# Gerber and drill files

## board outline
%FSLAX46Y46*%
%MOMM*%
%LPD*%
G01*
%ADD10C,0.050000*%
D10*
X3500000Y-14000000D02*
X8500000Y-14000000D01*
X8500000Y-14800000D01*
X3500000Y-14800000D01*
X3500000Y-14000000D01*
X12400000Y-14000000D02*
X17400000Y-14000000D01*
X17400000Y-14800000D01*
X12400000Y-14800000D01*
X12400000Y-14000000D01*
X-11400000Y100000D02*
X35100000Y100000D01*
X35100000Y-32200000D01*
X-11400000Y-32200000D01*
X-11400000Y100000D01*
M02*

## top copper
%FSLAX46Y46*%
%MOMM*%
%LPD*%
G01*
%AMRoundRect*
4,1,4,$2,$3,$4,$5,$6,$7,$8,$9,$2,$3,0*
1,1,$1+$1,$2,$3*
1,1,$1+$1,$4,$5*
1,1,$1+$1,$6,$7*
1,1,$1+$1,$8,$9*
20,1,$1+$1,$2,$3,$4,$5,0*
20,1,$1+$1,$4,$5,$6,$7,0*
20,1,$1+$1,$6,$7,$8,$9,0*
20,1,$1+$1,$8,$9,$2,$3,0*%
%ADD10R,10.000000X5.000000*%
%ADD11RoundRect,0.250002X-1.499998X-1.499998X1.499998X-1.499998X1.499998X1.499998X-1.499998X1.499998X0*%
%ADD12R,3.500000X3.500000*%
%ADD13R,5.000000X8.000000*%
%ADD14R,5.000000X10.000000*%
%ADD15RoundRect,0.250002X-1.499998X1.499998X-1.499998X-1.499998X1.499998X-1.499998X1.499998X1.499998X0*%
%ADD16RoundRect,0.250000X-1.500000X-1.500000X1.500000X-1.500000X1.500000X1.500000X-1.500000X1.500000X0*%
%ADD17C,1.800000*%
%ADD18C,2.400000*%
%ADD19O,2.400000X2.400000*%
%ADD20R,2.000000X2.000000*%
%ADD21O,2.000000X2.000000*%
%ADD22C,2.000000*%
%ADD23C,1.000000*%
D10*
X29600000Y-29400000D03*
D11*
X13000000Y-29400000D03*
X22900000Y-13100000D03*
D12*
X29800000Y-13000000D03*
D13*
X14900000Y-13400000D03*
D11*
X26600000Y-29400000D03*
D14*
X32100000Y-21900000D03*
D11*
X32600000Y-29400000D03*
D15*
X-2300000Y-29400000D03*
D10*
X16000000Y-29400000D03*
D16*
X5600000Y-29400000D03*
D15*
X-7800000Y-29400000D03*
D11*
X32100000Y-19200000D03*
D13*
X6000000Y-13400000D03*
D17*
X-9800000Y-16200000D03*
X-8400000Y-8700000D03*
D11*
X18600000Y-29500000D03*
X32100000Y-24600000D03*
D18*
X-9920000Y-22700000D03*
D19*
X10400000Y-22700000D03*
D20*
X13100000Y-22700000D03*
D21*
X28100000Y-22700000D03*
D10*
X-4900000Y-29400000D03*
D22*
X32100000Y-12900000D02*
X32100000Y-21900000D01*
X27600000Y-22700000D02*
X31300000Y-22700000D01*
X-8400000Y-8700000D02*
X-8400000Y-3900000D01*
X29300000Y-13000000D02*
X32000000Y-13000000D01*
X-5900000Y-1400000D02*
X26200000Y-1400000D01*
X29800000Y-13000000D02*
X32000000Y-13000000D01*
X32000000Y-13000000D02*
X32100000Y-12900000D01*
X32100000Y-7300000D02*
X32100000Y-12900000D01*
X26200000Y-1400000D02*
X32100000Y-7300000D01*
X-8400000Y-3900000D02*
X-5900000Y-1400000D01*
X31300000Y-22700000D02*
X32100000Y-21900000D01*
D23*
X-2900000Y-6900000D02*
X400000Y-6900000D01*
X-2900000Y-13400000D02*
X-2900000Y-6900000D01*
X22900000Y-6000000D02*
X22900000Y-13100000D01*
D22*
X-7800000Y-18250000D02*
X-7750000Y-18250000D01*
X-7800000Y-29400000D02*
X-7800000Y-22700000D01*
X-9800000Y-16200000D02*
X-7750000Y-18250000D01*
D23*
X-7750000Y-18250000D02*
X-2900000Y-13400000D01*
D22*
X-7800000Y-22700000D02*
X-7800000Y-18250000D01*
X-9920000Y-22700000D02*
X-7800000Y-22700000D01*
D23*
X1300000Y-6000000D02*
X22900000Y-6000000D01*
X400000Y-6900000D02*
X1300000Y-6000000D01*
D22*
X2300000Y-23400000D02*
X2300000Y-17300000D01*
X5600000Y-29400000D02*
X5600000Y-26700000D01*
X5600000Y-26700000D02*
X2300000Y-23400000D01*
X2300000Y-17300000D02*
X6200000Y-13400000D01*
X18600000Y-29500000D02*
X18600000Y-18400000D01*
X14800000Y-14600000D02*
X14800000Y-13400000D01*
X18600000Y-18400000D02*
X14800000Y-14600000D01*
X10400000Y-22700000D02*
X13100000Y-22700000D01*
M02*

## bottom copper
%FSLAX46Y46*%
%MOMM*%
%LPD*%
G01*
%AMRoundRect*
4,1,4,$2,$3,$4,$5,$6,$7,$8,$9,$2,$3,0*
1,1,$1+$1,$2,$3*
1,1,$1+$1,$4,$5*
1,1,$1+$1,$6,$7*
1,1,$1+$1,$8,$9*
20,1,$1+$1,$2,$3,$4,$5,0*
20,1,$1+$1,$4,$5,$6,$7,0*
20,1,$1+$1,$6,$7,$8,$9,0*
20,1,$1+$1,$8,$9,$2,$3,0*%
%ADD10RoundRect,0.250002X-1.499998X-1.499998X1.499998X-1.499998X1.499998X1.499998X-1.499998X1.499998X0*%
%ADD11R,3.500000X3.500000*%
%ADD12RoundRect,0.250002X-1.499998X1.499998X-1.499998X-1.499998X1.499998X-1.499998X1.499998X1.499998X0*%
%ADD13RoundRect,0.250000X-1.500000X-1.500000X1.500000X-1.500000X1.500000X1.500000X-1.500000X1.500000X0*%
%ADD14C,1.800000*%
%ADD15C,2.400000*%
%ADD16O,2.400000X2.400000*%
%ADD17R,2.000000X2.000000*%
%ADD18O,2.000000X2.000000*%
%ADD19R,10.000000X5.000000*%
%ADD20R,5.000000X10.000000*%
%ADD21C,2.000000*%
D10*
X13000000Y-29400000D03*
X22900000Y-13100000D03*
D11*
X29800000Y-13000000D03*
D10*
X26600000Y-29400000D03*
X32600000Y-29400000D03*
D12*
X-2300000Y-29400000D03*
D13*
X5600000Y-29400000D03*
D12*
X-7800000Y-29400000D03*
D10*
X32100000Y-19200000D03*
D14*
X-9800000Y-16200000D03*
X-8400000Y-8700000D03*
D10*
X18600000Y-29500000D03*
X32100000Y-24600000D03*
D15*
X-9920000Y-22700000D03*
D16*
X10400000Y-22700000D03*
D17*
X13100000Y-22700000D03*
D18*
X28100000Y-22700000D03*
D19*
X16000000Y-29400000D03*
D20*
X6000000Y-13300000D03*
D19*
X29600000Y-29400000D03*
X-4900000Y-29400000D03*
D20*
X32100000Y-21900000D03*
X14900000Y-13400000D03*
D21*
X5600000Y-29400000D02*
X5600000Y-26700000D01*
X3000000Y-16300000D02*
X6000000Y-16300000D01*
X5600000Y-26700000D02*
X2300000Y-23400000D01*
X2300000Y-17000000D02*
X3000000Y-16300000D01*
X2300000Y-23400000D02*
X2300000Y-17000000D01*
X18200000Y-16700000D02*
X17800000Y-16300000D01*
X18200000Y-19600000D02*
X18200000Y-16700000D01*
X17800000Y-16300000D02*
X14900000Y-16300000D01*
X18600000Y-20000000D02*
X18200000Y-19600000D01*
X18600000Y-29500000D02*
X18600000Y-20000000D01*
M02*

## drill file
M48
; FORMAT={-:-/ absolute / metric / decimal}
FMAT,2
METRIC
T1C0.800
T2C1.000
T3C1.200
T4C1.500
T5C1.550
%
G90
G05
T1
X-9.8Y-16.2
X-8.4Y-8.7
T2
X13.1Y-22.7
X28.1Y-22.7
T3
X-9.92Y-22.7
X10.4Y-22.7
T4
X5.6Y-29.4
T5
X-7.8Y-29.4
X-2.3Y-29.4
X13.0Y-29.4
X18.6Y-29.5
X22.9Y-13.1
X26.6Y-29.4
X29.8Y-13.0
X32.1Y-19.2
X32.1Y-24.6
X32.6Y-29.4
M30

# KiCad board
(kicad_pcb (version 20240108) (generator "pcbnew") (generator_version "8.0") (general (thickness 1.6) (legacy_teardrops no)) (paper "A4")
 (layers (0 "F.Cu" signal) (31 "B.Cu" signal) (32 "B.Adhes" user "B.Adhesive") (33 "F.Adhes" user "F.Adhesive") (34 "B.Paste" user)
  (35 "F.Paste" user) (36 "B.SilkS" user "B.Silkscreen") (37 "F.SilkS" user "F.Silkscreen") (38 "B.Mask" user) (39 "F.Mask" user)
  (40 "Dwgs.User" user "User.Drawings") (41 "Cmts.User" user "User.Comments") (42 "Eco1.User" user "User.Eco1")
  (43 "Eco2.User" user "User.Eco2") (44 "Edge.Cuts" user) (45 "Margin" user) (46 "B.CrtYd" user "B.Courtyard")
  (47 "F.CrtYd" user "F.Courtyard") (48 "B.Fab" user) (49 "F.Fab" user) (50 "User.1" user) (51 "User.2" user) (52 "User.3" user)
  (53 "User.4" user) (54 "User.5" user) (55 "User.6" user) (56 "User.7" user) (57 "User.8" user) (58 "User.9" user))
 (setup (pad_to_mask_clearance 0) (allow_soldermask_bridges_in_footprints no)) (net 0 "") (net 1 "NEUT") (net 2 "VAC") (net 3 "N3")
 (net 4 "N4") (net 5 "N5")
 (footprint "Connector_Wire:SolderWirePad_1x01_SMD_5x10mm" (layer "F.Cu") (at 29.6 29.4 -90)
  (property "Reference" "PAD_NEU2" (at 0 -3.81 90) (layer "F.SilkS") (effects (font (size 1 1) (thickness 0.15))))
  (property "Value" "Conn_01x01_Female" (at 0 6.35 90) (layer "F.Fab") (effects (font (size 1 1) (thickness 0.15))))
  (pad "1" smd rect (at 0 0 270) (size 5 10) (layers "F.Cu" "F.Paste" "F.Mask") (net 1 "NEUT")))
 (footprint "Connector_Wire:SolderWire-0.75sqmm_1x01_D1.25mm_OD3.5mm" (layer "F.Cu") (at 13 29.4)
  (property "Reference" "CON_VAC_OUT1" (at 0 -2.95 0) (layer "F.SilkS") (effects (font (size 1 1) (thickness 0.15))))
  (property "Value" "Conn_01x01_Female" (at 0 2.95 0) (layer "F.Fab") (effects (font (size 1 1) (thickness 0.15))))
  (pad "1" thru_hole roundrect (at 0 0) (size 3.5 3.5) (drill 1.55) (layers "*.Cu" "*.Mask") (remove_unused_layers no)
   (roundrect_rratio 0.071429) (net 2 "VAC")))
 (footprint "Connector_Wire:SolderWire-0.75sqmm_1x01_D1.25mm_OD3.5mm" (layer "F.Cu") (at 22.9 13.1)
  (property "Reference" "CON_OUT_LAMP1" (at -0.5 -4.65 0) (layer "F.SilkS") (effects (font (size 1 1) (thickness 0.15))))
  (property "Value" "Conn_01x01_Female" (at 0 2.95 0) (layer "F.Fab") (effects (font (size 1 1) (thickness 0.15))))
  (pad "1" thru_hole roundrect (at 0 0) (size 3.5 3.5) (drill 1.55) (layers "*.Cu" "*.Mask") (remove_unused_layers no)
   (roundrect_rratio 0.071429) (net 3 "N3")))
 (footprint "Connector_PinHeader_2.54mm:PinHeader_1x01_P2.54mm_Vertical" (layer "F.Cu") (at 29.8 13)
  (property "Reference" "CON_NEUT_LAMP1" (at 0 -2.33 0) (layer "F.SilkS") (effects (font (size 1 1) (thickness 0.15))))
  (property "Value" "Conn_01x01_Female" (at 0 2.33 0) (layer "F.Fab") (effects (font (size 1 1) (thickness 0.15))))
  (pad "1" thru_hole rect (at 0 0) (size 3.5 3.5) (drill 1.55) (layers "*.Cu" "*.Mask") (remove_unused_layers no) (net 1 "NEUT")))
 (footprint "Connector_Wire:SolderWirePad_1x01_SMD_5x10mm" (layer "F.Cu") (at 14.9 13.4)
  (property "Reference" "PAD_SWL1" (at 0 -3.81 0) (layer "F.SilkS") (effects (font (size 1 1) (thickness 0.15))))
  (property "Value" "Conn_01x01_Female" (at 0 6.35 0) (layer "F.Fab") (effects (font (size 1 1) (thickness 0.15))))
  (pad "1" smd rect (at 0 0) (size 5 8) (layers "F.Cu" "F.Paste" "F.Mask") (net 2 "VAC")))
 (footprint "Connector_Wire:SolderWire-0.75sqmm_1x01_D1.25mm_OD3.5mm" (layer "F.Cu") (at 26.6 29.4)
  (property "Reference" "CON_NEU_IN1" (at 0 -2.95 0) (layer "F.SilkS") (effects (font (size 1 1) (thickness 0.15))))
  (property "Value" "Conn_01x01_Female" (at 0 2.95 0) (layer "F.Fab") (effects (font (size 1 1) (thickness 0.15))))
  (pad "1" thru_hole roundrect (at 0 0) (size 3.5 3.5) (drill 1.55) (layers "*.Cu" "*.Mask") (remove_unused_layers no)
   (roundrect_rratio 0.071429) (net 1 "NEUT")))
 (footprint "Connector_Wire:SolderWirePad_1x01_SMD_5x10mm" (layer "F.Cu") (at 32.1 21.9)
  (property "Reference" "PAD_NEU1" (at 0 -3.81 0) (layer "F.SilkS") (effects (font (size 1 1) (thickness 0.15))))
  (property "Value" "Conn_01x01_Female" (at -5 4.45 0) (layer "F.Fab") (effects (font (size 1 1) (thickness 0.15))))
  (pad "1" smd rect (at 0 0) (size 5 10) (layers "F.Cu" "F.Paste" "F.Mask") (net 1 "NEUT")))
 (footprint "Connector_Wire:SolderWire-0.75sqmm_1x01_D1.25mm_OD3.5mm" (layer "F.Cu") (at 32.6 29.4)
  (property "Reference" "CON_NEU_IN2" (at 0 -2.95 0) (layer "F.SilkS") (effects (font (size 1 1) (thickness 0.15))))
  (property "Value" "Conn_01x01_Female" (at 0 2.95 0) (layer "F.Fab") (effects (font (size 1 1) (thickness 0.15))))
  (pad "1" thru_hole roundrect (at 0 0) (size 3.5 3.5) (drill 1.55) (layers "*.Cu" "*.Mask") (remove_unused_layers no)
   (roundrect_rratio 0.071429) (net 1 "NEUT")))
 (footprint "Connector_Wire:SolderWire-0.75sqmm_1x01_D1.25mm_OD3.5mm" (layer "F.Cu") (at -2.3 29.4 -90)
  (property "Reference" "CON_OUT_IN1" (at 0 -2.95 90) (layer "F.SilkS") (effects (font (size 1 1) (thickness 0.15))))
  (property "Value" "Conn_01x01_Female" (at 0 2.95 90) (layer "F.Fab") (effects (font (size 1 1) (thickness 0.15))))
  (pad "1" thru_hole roundrect (at 0 0 270) (size 3.5 3.5) (drill 1.55) (layers "*.Cu" "*.Mask") (remove_unused_layers no)
   (roundrect_rratio 0.071429) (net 3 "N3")))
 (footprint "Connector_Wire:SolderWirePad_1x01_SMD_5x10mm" (layer "F.Cu") (at 16 29.4 -90)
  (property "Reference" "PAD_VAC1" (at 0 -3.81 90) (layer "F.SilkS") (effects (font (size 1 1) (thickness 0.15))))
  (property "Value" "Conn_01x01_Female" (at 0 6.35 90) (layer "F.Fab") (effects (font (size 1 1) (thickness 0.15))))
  (pad "1" smd rect (at 0 0 270) (size 5 10) (layers "F.Cu" "F.Paste" "F.Mask") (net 2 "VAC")))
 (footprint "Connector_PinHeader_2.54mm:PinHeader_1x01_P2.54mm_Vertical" (layer "F.Cu") (at 5.6 29.4)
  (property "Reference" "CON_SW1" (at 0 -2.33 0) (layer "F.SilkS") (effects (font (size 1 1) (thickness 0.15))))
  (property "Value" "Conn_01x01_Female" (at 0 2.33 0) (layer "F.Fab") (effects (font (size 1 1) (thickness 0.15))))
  (pad "1" thru_hole roundrect (at 0 0) (size 3.5 3.5) (drill 1.5) (layers "*.Cu" "*.Mask") (remove_unused_layers no)
   (roundrect_rratio 0.07142857143) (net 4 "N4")))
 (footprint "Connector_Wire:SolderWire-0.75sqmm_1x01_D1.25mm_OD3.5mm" (layer "F.Cu") (at -7.8 29.4 -90)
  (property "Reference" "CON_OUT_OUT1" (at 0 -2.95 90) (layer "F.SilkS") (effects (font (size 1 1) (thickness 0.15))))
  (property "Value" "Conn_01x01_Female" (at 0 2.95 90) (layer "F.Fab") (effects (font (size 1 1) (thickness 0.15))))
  (pad "1" thru_hole roundrect (at 0 0 270) (size 3.5 3.5) (drill 1.55) (layers "*.Cu" "*.Mask") (remove_unused_layers no)
   (roundrect_rratio 0.071429) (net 3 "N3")))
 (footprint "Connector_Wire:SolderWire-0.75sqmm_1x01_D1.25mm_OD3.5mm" (layer "F.Cu") (at 32.1 19.2)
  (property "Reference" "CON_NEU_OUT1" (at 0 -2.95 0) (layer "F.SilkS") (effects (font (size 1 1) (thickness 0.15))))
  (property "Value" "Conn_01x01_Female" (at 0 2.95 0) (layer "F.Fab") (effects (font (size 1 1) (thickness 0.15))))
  (pad "1" thru_hole roundrect (at 0 0) (size 3.5 3.5) (drill 1.55) (layers "*.Cu" "*.Mask") (remove_unused_layers no)
   (roundrect_rratio 0.071429) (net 1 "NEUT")))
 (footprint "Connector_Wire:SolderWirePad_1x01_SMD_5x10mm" (layer "F.Cu") (at 6 13.4)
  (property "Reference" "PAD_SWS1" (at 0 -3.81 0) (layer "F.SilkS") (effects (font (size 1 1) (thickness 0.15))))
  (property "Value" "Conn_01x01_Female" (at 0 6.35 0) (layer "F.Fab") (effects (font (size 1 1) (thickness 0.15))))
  (pad "1" smd rect (at 0 0) (size 5 8) (layers "F.Cu" "F.Paste" "F.Mask") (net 4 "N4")))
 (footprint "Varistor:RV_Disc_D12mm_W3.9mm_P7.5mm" (layer "F.Cu") (at -9.8 16.2 90)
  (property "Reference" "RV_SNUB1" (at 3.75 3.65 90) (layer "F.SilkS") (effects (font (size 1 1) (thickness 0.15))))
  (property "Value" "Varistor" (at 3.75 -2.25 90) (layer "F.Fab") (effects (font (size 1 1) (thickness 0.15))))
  (pad "1" thru_hole circle (at 0 0 90) (size 1.8 1.8) (drill 0.8) (layers "*.Cu" "*.Mask") (remove_unused_layers no) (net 3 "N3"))
  (pad "2" thru_hole circle (at 7.5 1.4 90) (size 1.8 1.8) (drill 0.8) (layers "*.Cu" "*.Mask") (remove_unused_layers no) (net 1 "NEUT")))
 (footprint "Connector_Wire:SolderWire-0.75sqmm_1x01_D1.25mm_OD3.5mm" (layer "F.Cu") (at 18.6 29.5)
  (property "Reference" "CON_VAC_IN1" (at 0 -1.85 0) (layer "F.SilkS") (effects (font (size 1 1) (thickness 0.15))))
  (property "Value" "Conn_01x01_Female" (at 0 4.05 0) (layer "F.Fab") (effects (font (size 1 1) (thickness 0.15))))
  (pad "1" thru_hole roundrect (at 0 0) (size 3.5 3.5) (drill 1.55) (layers "*.Cu" "*.Mask") (remove_unused_layers no)
   (roundrect_rratio 0.071429) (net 2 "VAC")))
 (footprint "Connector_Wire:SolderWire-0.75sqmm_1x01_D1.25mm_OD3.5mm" (layer "F.Cu") (at 32.1 24.6)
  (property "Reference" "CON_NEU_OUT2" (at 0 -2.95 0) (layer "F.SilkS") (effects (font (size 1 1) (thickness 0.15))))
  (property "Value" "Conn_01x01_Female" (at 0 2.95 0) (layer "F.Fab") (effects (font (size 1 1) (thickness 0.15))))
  (pad "1" thru_hole roundrect (at 0 0) (size 3.5 3.5) (drill 1.55) (layers "*.Cu" "*.Mask") (remove_unused_layers no)
   (roundrect_rratio 0.071429) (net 1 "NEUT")))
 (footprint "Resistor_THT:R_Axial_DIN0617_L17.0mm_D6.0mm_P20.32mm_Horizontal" (layer "F.Cu") (at -9.92 22.7)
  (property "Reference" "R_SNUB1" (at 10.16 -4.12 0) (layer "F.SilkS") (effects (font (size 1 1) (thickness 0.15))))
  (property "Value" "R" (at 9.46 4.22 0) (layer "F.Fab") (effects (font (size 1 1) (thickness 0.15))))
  (pad "1" thru_hole circle (at 0 0) (size 2.4 2.4) (drill 1.2) (layers "*.Cu" "*.Mask") (remove_unused_layers no) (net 3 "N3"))
  (pad "2" thru_hole oval (at 20.32 0) (size 2.4 2.4) (drill 1.2) (layers "*.Cu" "*.Mask") (remove_unused_layers no) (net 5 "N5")))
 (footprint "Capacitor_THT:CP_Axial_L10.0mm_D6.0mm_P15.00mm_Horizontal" (layer "F.Cu") (at 13.1 22.7)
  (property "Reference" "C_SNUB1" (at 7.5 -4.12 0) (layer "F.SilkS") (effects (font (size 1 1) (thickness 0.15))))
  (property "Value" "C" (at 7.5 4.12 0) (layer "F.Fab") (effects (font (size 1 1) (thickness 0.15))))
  (pad "1" thru_hole rect (at 0 0) (size 2 2) (drill 1) (layers "*.Cu" "*.Mask") (remove_unused_layers no) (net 5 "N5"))
  (pad "2" thru_hole oval (at 15 0) (size 2 2) (drill 1) (layers "*.Cu" "*.Mask") (remove_unused_layers no) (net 1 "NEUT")))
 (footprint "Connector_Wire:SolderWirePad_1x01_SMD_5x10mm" (layer "F.Cu") (at -4.9 29.4 -90)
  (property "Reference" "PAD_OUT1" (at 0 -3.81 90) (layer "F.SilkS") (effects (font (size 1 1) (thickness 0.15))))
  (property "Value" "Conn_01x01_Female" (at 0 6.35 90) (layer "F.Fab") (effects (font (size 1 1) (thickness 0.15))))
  (pad "1" smd rect (at 0 0 270) (size 5 10) (layers "F.Cu" "F.Paste" "F.Mask") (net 3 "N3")))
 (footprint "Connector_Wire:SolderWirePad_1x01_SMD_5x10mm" (layer "B.Cu") (at 16 29.4 -90)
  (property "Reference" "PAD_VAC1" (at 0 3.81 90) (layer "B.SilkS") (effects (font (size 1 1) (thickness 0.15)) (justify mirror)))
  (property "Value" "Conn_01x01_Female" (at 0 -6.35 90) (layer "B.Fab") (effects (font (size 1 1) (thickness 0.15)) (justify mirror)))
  (pad "1" smd rect (at 0 0 270) (size 5 10) (layers "B.Cu" "B.Paste" "B.Mask")))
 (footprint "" (layer "B.Cu") (at 6 13.3 180)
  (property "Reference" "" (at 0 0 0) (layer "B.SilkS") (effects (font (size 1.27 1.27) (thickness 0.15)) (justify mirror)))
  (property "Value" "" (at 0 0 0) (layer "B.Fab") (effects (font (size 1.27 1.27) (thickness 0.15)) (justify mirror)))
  (pad "1" smd rect (at 0 0 180) (size 5 10) (layers "B.Cu" "B.Paste" "B.Mask") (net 4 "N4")))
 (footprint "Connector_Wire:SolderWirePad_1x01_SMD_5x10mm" (layer "B.Cu") (at 29.6 29.4 -90)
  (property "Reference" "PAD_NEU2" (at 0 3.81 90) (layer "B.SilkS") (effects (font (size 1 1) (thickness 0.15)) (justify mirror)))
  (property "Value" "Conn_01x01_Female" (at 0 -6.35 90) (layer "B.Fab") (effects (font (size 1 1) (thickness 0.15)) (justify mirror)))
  (pad "1" smd rect (at 0 0 270) (size 5 10) (layers "B.Cu" "B.Paste" "B.Mask")))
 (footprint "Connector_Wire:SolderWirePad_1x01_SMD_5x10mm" (layer "B.Cu") (at -4.9 29.4 -90)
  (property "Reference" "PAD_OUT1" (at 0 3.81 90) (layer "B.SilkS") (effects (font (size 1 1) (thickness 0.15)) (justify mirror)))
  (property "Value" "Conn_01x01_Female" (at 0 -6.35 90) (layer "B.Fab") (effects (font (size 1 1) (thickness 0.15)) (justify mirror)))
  (pad "1" smd rect (at 0 0 270) (size 5 10) (layers "B.Cu" "B.Paste" "B.Mask")))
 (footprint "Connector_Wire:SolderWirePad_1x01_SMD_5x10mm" (layer "B.Cu") (at 32.1 21.9 180)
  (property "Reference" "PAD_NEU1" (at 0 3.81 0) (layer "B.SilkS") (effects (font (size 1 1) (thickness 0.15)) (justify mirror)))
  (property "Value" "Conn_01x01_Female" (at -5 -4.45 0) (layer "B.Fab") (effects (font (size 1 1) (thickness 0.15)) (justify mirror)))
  (pad "1" smd rect (at 0 0 180) (size 5 10) (layers "B.Cu" "B.Paste" "B.Mask")))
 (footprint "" (layer "B.Cu") (at 14.9 13.4 180)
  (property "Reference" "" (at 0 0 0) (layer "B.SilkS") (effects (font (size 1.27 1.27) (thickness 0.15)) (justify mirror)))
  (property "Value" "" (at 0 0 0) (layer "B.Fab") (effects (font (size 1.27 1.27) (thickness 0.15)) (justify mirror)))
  (pad "1" smd rect (at 0 0 180) (size 5 10) (layers "B.Cu" "B.Paste" "B.Mask") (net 2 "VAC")))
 (gr_rect (start 3.5 14) (end 8.5 14.8) (stroke (width 0.05) (type default)) (fill none) (layer "Edge.Cuts"))
 (gr_rect (start 12.4 14) (end 17.4 14.8) (stroke (width 0.05) (type default)) (fill none) (layer "Edge.Cuts"))
 (gr_rect (start -11.4 -0.1) (end 35.1 32.2) (stroke (width 0.05) (type default)) (fill none) (layer "Edge.Cuts"))
 (segment (start 32.1 12.9) (end 32.1 21.9) (width 2) (layer "F.Cu") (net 1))
 (segment (start 27.6 22.7) (end 31.3 22.7) (width 2) (layer "F.Cu") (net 1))
 (segment (start -8.4 8.7) (end -8.4 3.9) (width 2) (layer "F.Cu") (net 1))
 (segment (start 29.3 13) (end 32 13) (width 2) (layer "F.Cu") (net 1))
 (segment (start -5.9 1.4) (end 26.2 1.4) (width 2) (layer "F.Cu") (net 1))
 (segment (start 29.8 13) (end 32 13) (width 2) (layer "F.Cu") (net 1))
 (segment (start 32 13) (end 32.1 12.9) (width 2) (layer "F.Cu") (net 1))
 (segment (start 32.1 7.3) (end 32.1 12.9) (width 2) (layer "F.Cu") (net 1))
 (segment (start 26.2 1.4) (end 32.1 7.3) (width 2) (layer "F.Cu") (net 1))
 (segment (start -8.4 3.9) (end -5.9 1.4) (width 2) (layer "F.Cu") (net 1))
 (segment (start 31.3 22.7) (end 32.1 21.9) (width 2) (layer "F.Cu") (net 1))
 (segment (start -2.9 6.9) (end 0.4 6.9) (width 1) (layer "F.Cu") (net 3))
 (segment (start -2.9 13.4) (end -2.9 6.9) (width 1) (layer "F.Cu") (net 3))
 (segment (start 22.9 6) (end 22.9 13.1) (width 1) (layer "F.Cu") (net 3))
 (segment (start -7.8 18.25) (end -7.75 18.25) (width 2) (layer "F.Cu") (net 3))
 (segment (start -7.8 29.4) (end -7.8 22.7) (width 2) (layer "F.Cu") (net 3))
 (segment (start -9.8 16.2) (end -7.75 18.25) (width 2) (layer "F.Cu") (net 3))
 (segment (start -7.75 18.25) (end -2.9 13.4) (width 1) (layer "F.Cu") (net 3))
 (segment (start -7.8 22.7) (end -7.8 18.25) (width 2) (layer "F.Cu") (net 3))
 (segment (start -9.92 22.7) (end -7.8 22.7) (width 2) (layer "F.Cu") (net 3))
 (segment (start 1.3 6) (end 22.9 6) (width 1) (layer "F.Cu") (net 3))
 (segment (start 0.4 6.9) (end 1.3 6) (width 1) (layer "F.Cu") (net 3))
 (segment (start 2.3 23.4) (end 2.3 17.3) (width 2) (layer "F.Cu") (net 4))
 (segment (start 5.6 29.4) (end 5.6 26.7) (width 2) (layer "F.Cu") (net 4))
 (segment (start 5.6 26.7) (end 2.3 23.4) (width 2) (layer "F.Cu") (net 4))
 (segment (start 2.3 17.3) (end 6.2 13.4) (width 2) (layer "F.Cu") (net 4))
 (segment (start 5.6 29.4) (end 5.6 26.7) (width 2) (layer "B.Cu") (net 4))
 (segment (start 3 16.3) (end 6 16.3) (width 2) (layer "B.Cu") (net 4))
 (segment (start 5.6 26.7) (end 2.3 23.4) (width 2) (layer "B.Cu") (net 4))
 (segment (start 2.3 17) (end 3 16.3) (width 2) (layer "B.Cu") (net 4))
 (segment (start 2.3 23.4) (end 2.3 17) (width 2) (layer "B.Cu") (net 4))
 (segment (start 18.6 29.5) (end 18.6 18.4) (width 2) (layer "F.Cu") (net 2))
 (segment (start 14.8 14.6) (end 14.8 13.4) (width 2) (layer "F.Cu") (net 2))
 (segment (start 18.6 18.4) (end 14.8 14.6) (width 2) (layer "F.Cu") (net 2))
 (segment (start 18.2 16.7) (end 17.8 16.3) (width 2) (layer "B.Cu") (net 2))
 (segment (start 18.2 19.6) (end 18.2 16.7) (width 2) (layer "B.Cu") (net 2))
 (segment (start 17.8 16.3) (end 14.9 16.3) (width 2) (layer "B.Cu") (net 2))
 (segment (start 18.6 20) (end 18.2 19.6) (width 2) (layer "B.Cu") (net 2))
 (segment (start 18.6 29.5) (end 18.6 20) (width 2) (layer "B.Cu") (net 2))
 (segment (start 10.4 22.7) (end 13.1 22.7) (width 2) (layer "F.Cu") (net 5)))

